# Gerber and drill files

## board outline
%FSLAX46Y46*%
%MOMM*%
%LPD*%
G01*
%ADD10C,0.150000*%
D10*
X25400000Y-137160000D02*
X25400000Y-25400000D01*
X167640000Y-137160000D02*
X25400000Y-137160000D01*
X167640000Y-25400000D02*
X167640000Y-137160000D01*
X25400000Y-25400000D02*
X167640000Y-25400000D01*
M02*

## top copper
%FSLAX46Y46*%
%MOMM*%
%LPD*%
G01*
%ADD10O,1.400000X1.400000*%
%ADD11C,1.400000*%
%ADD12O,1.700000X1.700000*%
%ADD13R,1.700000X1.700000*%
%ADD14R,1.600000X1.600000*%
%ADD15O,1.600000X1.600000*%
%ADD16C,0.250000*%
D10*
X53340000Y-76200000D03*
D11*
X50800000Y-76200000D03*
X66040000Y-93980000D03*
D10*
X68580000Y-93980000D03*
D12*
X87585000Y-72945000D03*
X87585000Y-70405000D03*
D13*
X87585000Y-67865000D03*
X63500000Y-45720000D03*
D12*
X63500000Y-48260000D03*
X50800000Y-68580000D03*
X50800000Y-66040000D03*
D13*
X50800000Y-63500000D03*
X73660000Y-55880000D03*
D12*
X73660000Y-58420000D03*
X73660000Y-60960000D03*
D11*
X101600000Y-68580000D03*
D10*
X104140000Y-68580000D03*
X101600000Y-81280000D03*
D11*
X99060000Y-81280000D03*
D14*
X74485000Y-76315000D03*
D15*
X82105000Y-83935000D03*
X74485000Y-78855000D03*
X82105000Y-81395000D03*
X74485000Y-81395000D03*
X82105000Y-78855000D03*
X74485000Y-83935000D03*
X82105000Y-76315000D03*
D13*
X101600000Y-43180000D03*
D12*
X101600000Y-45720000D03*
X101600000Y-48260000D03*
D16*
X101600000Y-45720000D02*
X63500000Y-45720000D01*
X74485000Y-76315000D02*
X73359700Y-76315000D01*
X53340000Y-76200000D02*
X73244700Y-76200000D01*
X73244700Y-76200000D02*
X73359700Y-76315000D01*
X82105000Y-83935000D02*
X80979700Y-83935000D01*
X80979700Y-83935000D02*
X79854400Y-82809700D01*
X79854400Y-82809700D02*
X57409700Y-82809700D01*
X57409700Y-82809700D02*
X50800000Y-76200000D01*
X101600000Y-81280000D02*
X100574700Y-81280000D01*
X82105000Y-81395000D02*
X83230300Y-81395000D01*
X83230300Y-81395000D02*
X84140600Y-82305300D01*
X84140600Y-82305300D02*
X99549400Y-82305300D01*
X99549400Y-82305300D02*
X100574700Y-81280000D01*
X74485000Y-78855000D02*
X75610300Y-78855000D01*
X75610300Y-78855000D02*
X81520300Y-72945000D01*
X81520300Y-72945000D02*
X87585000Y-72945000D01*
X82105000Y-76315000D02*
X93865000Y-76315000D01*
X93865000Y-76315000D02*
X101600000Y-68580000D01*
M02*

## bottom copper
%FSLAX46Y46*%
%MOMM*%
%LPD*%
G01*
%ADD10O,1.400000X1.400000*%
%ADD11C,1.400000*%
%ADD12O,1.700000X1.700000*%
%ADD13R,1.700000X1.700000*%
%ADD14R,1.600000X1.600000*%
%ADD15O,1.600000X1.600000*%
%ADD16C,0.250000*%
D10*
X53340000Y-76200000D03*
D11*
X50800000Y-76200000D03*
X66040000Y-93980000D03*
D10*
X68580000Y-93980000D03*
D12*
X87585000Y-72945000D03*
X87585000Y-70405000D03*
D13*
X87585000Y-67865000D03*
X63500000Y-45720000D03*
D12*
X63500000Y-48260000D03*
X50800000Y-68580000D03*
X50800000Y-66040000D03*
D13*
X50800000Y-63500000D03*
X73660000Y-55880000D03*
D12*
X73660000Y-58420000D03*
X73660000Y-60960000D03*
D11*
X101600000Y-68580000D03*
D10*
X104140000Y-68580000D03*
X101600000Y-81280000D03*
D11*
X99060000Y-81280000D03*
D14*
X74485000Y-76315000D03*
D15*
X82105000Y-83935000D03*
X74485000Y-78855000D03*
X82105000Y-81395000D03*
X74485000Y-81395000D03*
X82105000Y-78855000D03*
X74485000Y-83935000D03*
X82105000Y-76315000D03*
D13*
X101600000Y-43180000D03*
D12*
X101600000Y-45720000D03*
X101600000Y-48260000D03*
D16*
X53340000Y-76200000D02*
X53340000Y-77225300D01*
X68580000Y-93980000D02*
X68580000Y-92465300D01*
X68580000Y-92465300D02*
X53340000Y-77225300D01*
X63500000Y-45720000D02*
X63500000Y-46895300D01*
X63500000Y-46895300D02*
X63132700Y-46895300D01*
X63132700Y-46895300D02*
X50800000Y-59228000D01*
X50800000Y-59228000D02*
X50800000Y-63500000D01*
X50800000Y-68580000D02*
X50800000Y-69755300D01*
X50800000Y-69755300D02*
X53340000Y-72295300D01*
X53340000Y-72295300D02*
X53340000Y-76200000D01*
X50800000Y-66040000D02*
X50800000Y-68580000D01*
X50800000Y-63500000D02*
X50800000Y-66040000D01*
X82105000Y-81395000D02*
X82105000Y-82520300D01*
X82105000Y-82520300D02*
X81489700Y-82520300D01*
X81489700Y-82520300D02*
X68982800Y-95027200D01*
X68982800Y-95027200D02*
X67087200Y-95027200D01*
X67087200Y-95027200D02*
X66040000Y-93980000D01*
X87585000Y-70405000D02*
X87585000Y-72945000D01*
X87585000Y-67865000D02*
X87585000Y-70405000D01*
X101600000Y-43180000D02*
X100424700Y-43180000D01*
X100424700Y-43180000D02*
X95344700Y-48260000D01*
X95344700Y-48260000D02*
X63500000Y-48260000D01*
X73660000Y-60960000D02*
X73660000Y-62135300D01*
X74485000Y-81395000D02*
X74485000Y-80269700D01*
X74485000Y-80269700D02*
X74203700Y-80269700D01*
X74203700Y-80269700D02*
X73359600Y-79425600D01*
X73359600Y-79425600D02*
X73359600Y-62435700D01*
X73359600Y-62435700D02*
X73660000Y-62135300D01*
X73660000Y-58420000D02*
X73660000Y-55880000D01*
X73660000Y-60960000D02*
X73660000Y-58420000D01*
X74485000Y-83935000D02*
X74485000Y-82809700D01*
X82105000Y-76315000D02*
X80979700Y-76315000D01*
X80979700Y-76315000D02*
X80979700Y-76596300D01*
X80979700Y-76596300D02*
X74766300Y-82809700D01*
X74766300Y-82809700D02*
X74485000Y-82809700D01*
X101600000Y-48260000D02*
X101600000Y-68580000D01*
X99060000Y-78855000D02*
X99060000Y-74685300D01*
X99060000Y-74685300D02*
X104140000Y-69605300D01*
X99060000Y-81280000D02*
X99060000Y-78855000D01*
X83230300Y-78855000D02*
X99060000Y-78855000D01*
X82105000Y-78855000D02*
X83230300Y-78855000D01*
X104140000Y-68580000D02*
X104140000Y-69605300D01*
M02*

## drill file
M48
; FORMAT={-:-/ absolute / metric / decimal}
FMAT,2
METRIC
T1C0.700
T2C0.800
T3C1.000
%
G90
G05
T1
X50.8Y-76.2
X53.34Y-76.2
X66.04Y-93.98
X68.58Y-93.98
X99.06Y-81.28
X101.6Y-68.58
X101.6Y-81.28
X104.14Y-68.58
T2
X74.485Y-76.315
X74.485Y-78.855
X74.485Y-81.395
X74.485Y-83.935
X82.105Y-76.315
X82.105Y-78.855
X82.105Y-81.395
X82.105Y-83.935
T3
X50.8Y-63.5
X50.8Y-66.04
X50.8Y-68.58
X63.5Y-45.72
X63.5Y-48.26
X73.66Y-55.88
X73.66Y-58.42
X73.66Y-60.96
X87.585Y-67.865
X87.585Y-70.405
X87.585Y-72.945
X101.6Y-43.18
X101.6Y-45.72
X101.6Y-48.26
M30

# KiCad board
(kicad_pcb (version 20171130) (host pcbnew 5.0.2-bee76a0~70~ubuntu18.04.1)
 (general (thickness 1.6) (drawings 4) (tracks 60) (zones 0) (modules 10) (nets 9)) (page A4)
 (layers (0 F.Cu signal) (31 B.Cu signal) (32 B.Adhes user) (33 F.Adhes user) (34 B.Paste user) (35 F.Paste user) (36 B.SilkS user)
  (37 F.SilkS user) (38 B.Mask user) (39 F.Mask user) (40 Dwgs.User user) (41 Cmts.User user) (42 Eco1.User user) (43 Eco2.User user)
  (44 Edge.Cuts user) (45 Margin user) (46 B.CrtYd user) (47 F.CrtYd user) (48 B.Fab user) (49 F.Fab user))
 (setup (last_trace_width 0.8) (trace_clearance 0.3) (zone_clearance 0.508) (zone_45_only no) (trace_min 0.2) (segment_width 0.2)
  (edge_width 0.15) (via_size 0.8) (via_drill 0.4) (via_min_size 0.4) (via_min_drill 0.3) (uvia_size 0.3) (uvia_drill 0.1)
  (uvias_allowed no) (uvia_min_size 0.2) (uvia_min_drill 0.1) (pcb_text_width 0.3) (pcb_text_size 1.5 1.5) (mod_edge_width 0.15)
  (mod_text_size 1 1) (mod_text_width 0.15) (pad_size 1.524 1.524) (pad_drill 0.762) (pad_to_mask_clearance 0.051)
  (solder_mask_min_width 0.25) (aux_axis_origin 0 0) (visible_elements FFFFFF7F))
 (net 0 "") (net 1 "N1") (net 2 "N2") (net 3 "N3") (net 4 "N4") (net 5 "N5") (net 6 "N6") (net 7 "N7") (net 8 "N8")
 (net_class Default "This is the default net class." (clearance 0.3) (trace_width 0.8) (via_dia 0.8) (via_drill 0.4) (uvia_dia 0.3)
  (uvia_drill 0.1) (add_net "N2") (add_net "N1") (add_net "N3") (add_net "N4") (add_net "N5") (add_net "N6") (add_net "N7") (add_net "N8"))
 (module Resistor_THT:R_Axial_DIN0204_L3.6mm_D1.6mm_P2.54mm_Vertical (layer F.Cu) (at 50.8 76.2)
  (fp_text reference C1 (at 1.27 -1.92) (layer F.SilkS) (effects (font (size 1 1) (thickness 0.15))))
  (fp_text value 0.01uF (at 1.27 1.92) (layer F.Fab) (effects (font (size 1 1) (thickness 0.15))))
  (pad 2 thru_hole oval (at 2.54 0) (size 1.4 1.4) (drill 0.7) (layers *.Cu *.Mask) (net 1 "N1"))
  (pad 1 thru_hole circle (at 0 0) (size 1.4 1.4) (drill 0.7) (layers *.Cu *.Mask) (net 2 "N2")))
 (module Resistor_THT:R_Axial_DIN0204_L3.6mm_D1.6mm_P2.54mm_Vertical (layer F.Cu) (at 66.04 93.98)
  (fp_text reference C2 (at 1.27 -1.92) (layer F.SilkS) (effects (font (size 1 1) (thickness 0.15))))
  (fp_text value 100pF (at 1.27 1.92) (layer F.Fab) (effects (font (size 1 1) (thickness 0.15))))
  (pad 1 thru_hole circle (at 0 0) (size 1.4 1.4) (drill 0.7) (layers *.Cu *.Mask) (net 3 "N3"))
  (pad 2 thru_hole oval (at 2.54 0) (size 1.4 1.4) (drill 0.7) (layers *.Cu *.Mask) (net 1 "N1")))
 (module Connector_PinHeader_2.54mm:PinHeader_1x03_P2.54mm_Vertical (layer F.Cu) (at 87.585 67.865)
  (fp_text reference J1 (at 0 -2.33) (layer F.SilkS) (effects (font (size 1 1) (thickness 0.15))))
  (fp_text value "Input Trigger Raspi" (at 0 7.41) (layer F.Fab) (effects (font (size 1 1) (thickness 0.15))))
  (pad 3 thru_hole oval (at 0 5.08) (size 1.7 1.7) (drill 1) (layers *.Cu *.Mask) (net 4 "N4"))
  (pad 2 thru_hole oval (at 0 2.54) (size 1.7 1.7) (drill 1) (layers *.Cu *.Mask) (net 4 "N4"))
  (pad 1 thru_hole rect (at 0 0) (size 1.7 1.7) (drill 1) (layers *.Cu *.Mask) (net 4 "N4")))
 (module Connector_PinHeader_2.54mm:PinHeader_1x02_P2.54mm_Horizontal (layer F.Cu) (at 63.5 45.72)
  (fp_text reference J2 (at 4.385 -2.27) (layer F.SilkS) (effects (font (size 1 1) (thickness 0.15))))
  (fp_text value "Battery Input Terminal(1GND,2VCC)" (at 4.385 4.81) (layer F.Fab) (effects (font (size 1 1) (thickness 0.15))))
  (pad 1 thru_hole rect (at 0 0) (size 1.7 1.7) (drill 1) (layers *.Cu *.Mask) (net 1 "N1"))
  (pad 2 thru_hole oval (at 0 2.54) (size 1.7 1.7) (drill 1) (layers *.Cu *.Mask) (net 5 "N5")))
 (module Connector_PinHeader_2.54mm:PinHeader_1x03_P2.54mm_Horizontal (layer F.Cu) (at 50.8 63.5)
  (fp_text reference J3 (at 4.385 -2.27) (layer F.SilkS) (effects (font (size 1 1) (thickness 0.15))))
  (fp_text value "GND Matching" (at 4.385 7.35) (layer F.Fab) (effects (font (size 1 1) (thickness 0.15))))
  (pad 3 thru_hole oval (at 0 5.08) (size 1.7 1.7) (drill 1) (layers *.Cu *.Mask) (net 1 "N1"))
  (pad 2 thru_hole oval (at 0 2.54) (size 1.7 1.7) (drill 1) (layers *.Cu *.Mask) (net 1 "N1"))
  (pad 1 thru_hole rect (at 0 0) (size 1.7 1.7) (drill 1) (layers *.Cu *.Mask) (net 1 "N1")))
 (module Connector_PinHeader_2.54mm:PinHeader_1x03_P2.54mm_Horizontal (layer F.Cu) (at 73.66 55.88)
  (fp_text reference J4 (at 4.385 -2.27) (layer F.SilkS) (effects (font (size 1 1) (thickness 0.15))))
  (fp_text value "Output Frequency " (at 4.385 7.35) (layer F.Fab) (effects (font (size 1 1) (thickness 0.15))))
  (pad 1 thru_hole rect (at 0 0) (size 1.7 1.7) (drill 1) (layers *.Cu *.Mask) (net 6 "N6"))
  (pad 2 thru_hole oval (at 0 2.54) (size 1.7 1.7) (drill 1) (layers *.Cu *.Mask) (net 6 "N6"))
  (pad 3 thru_hole oval (at 0 5.08) (size 1.7 1.7) (drill 1) (layers *.Cu *.Mask) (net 6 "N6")))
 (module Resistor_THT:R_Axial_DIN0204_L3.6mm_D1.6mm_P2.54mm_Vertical (layer F.Cu) (at 101.6 68.58)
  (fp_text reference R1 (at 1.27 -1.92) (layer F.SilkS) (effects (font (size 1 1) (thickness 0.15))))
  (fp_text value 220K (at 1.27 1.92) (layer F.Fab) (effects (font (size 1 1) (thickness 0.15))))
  (pad 1 thru_hole circle (at 0 0) (size 1.4 1.4) (drill 0.7) (layers *.Cu *.Mask) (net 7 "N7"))
  (pad 2 thru_hole oval (at 2.54 0) (size 1.4 1.4) (drill 0.7) (layers *.Cu *.Mask) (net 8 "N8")))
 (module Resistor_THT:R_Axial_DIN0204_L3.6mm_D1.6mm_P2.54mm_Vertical (layer F.Cu) (at 99.06 81.28)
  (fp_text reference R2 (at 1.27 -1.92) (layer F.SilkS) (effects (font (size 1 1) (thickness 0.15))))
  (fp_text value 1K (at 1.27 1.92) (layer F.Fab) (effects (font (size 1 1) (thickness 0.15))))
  (pad 2 thru_hole oval (at 2.54 0) (size 1.4 1.4) (drill 0.7) (layers *.Cu *.Mask) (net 3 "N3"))
  (pad 1 thru_hole circle (at 0 0) (size 1.4 1.4) (drill 0.7) (layers *.Cu *.Mask) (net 8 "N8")))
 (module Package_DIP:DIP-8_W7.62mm (layer F.Cu) (at 74.485 76.315)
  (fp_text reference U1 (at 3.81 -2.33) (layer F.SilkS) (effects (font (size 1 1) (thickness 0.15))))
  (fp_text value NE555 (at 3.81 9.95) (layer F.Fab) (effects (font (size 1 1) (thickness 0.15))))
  (pad 1 thru_hole rect (at 0 0) (size 1.6 1.6) (drill 0.8) (layers *.Cu *.Mask) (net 1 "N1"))
  (pad 5 thru_hole oval (at 7.62 7.62) (size 1.6 1.6) (drill 0.8) (layers *.Cu *.Mask) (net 2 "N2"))
  (pad 2 thru_hole oval (at 0 2.54) (size 1.6 1.6) (drill 0.8) (layers *.Cu *.Mask) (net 4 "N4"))
  (pad 6 thru_hole oval (at 7.62 5.08) (size 1.6 1.6) (drill 0.8) (layers *.Cu *.Mask) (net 3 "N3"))
  (pad 3 thru_hole oval (at 0 5.08) (size 1.6 1.6) (drill 0.8) (layers *.Cu *.Mask) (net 6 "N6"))
  (pad 7 thru_hole oval (at 7.62 2.54) (size 1.6 1.6) (drill 0.8) (layers *.Cu *.Mask) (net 8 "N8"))
  (pad 4 thru_hole oval (at 0 7.62) (size 1.6 1.6) (drill 0.8) (layers *.Cu *.Mask) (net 7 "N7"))
  (pad 8 thru_hole oval (at 7.62 0) (size 1.6 1.6) (drill 0.8) (layers *.Cu *.Mask) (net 7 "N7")))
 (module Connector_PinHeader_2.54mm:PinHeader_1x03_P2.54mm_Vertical (layer F.Cu) (at 101.6 43.18)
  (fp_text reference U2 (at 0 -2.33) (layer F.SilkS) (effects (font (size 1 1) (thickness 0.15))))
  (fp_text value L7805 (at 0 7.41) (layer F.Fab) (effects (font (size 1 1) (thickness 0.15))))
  (pad 1 thru_hole rect (at 0 0) (size 1.7 1.7) (drill 1) (layers *.Cu *.Mask) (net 5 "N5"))
  (pad 2 thru_hole oval (at 0 2.54) (size 1.7 1.7) (drill 1) (layers *.Cu *.Mask) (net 1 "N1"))
  (pad 3 thru_hole oval (at 0 5.08) (size 1.7 1.7) (drill 1) (layers *.Cu *.Mask) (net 7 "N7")))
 (gr_line (start 25.4 137.16) (end 25.4 25.4) (angle 90) (layer Edge.Cuts) (width 0.15))
 (gr_line (start 167.64 137.16) (end 25.4 137.16) (angle 90) (layer Edge.Cuts) (width 0.15))
 (gr_line (start 167.64 25.4) (end 167.64 137.16) (angle 90) (layer Edge.Cuts) (width 0.15))
 (gr_line (start 25.4 25.4) (end 167.64 25.4) (angle 90) (layer Edge.Cuts) (width 0.15))
 (segment (start 101.6 45.72) (end 63.5 45.72) (width 0.25) (layer F.Cu) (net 1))
 (segment (start 74.485 76.315) (end 73.3597 76.315) (width 0.25) (layer F.Cu) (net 1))
 (segment (start 53.34 76.2) (end 73.2447 76.2) (width 0.25) (layer F.Cu) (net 1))
 (segment (start 73.2447 76.2) (end 73.3597 76.315) (width 0.25) (layer F.Cu) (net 1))
 (segment (start 53.34 76.2) (end 53.34 77.2253) (width 0.25) (layer B.Cu) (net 1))
 (segment (start 68.58 93.98) (end 68.58 92.4653) (width 0.25) (layer B.Cu) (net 1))
 (segment (start 68.58 92.4653) (end 53.34 77.2253) (width 0.25) (layer B.Cu) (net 1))
 (segment (start 63.5 45.72) (end 63.5 46.8953) (width 0.25) (layer B.Cu) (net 1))
 (segment (start 63.5 46.8953) (end 63.1327 46.8953) (width 0.25) (layer B.Cu) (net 1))
 (segment (start 63.1327 46.8953) (end 50.8 59.228) (width 0.25) (layer B.Cu) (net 1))
 (segment (start 50.8 59.228) (end 50.8 63.5) (width 0.25) (layer B.Cu) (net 1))
 (segment (start 50.8 68.58) (end 50.8 69.7553) (width 0.25) (layer B.Cu) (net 1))
 (segment (start 50.8 69.7553) (end 53.34 72.2953) (width 0.25) (layer B.Cu) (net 1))
 (segment (start 53.34 72.2953) (end 53.34 76.2) (width 0.25) (layer B.Cu) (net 1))
 (segment (start 50.8 66.04) (end 50.8 68.58) (width 0.25) (layer B.Cu) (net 1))
 (segment (start 50.8 63.5) (end 50.8 66.04) (width 0.25) (layer B.Cu) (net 1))
 (segment (start 82.105 83.935) (end 80.9797 83.935) (width 0.25) (layer F.Cu) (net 2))
 (segment (start 80.9797 83.935) (end 79.8544 82.8097) (width 0.25) (layer F.Cu) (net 2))
 (segment (start 79.8544 82.8097) (end 57.4097 82.8097) (width 0.25) (layer F.Cu) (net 2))
 (segment (start 57.4097 82.8097) (end 50.8 76.2) (width 0.25) (layer F.Cu) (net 2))
 (segment (start 82.105 81.395) (end 82.105 82.5203) (width 0.25) (layer B.Cu) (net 3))
 (segment (start 82.105 82.5203) (end 81.4897 82.5203) (width 0.25) (layer B.Cu) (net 3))
 (segment (start 81.4897 82.5203) (end 68.9828 95.0272) (width 0.25) (layer B.Cu) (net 3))
 (segment (start 68.9828 95.0272) (end 67.0872 95.0272) (width 0.25) (layer B.Cu) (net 3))
 (segment (start 67.0872 95.0272) (end 66.04 93.98) (width 0.25) (layer B.Cu) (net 3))
 (segment (start 101.6 81.28) (end 100.5747 81.28) (width 0.25) (layer F.Cu) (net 3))
 (segment (start 82.105 81.395) (end 83.2303 81.395) (width 0.25) (layer F.Cu) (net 3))
 (segment (start 83.2303 81.395) (end 84.1406 82.3053) (width 0.25) (layer F.Cu) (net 3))
 (segment (start 84.1406 82.3053) (end 99.5494 82.3053) (width 0.25) (layer F.Cu) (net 3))
 (segment (start 99.5494 82.3053) (end 100.5747 81.28) (width 0.25) (layer F.Cu) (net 3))
 (segment (start 87.585 70.405) (end 87.585 72.945) (width 0.25) (layer B.Cu) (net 4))
 (segment (start 87.585 67.865) (end 87.585 70.405) (width 0.25) (layer B.Cu) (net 4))
 (segment (start 74.485 78.855) (end 75.6103 78.855) (width 0.25) (layer F.Cu) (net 4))
 (segment (start 75.6103 78.855) (end 81.5203 72.945) (width 0.25) (layer F.Cu) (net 4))
 (segment (start 81.5203 72.945) (end 87.585 72.945) (width 0.25) (layer F.Cu) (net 4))
 (segment (start 101.6 43.18) (end 100.4247 43.18) (width 0.25) (layer B.Cu) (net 5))
 (segment (start 100.4247 43.18) (end 95.3447 48.26) (width 0.25) (layer B.Cu) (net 5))
 (segment (start 95.3447 48.26) (end 63.5 48.26) (width 0.25) (layer B.Cu) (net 5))
 (segment (start 73.66 60.96) (end 73.66 62.1353) (width 0.25) (layer B.Cu) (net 6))
 (segment (start 74.485 81.395) (end 74.485 80.2697) (width 0.25) (layer B.Cu) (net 6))
 (segment (start 74.485 80.2697) (end 74.2037 80.2697) (width 0.25) (layer B.Cu) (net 6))
 (segment (start 74.2037 80.2697) (end 73.3596 79.4256) (width 0.25) (layer B.Cu) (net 6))
 (segment (start 73.3596 79.4256) (end 73.3596 62.4357) (width 0.25) (layer B.Cu) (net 6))
 (segment (start 73.3596 62.4357) (end 73.66 62.1353) (width 0.25) (layer B.Cu) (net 6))
 (segment (start 73.66 58.42) (end 73.66 55.88) (width 0.25) (layer B.Cu) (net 6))
 (segment (start 73.66 60.96) (end 73.66 58.42) (width 0.25) (layer B.Cu) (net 6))
 (segment (start 74.485 83.935) (end 74.485 82.8097) (width 0.25) (layer B.Cu) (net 7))
 (segment (start 82.105 76.315) (end 80.9797 76.315) (width 0.25) (layer B.Cu) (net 7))
 (segment (start 80.9797 76.315) (end 80.9797 76.5963) (width 0.25) (layer B.Cu) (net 7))
 (segment (start 80.9797 76.5963) (end 74.7663 82.8097) (width 0.25) (layer B.Cu) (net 7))
 (segment (start 74.7663 82.8097) (end 74.485 82.8097) (width 0.25) (layer B.Cu) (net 7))
 (segment (start 82.105 76.315) (end 93.865 76.315) (width 0.25) (layer F.Cu) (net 7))
 (segment (start 93.865 76.315) (end 101.6 68.58) (width 0.25) (layer F.Cu) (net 7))
 (segment (start 101.6 48.26) (end 101.6 68.58) (width 0.25) (layer B.Cu) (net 7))
 (segment (start 99.06 78.855) (end 99.06 74.6853) (width 0.25) (layer B.Cu) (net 8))
 (segment (start 99.06 74.6853) (end 104.14 69.6053) (width 0.25) (layer B.Cu) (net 8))
 (segment (start 99.06 81.28) (end 99.06 78.855) (width 0.25) (layer B.Cu) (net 8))
 (segment (start 83.2303 78.855) (end 99.06 78.855) (width 0.25) (layer B.Cu) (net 8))
 (segment (start 82.105 78.855) (end 83.2303 78.855) (width 0.25) (layer B.Cu) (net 8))
 (segment (start 104.14 68.58) (end 104.14 69.6053) (width 0.25) (layer B.Cu) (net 8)))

